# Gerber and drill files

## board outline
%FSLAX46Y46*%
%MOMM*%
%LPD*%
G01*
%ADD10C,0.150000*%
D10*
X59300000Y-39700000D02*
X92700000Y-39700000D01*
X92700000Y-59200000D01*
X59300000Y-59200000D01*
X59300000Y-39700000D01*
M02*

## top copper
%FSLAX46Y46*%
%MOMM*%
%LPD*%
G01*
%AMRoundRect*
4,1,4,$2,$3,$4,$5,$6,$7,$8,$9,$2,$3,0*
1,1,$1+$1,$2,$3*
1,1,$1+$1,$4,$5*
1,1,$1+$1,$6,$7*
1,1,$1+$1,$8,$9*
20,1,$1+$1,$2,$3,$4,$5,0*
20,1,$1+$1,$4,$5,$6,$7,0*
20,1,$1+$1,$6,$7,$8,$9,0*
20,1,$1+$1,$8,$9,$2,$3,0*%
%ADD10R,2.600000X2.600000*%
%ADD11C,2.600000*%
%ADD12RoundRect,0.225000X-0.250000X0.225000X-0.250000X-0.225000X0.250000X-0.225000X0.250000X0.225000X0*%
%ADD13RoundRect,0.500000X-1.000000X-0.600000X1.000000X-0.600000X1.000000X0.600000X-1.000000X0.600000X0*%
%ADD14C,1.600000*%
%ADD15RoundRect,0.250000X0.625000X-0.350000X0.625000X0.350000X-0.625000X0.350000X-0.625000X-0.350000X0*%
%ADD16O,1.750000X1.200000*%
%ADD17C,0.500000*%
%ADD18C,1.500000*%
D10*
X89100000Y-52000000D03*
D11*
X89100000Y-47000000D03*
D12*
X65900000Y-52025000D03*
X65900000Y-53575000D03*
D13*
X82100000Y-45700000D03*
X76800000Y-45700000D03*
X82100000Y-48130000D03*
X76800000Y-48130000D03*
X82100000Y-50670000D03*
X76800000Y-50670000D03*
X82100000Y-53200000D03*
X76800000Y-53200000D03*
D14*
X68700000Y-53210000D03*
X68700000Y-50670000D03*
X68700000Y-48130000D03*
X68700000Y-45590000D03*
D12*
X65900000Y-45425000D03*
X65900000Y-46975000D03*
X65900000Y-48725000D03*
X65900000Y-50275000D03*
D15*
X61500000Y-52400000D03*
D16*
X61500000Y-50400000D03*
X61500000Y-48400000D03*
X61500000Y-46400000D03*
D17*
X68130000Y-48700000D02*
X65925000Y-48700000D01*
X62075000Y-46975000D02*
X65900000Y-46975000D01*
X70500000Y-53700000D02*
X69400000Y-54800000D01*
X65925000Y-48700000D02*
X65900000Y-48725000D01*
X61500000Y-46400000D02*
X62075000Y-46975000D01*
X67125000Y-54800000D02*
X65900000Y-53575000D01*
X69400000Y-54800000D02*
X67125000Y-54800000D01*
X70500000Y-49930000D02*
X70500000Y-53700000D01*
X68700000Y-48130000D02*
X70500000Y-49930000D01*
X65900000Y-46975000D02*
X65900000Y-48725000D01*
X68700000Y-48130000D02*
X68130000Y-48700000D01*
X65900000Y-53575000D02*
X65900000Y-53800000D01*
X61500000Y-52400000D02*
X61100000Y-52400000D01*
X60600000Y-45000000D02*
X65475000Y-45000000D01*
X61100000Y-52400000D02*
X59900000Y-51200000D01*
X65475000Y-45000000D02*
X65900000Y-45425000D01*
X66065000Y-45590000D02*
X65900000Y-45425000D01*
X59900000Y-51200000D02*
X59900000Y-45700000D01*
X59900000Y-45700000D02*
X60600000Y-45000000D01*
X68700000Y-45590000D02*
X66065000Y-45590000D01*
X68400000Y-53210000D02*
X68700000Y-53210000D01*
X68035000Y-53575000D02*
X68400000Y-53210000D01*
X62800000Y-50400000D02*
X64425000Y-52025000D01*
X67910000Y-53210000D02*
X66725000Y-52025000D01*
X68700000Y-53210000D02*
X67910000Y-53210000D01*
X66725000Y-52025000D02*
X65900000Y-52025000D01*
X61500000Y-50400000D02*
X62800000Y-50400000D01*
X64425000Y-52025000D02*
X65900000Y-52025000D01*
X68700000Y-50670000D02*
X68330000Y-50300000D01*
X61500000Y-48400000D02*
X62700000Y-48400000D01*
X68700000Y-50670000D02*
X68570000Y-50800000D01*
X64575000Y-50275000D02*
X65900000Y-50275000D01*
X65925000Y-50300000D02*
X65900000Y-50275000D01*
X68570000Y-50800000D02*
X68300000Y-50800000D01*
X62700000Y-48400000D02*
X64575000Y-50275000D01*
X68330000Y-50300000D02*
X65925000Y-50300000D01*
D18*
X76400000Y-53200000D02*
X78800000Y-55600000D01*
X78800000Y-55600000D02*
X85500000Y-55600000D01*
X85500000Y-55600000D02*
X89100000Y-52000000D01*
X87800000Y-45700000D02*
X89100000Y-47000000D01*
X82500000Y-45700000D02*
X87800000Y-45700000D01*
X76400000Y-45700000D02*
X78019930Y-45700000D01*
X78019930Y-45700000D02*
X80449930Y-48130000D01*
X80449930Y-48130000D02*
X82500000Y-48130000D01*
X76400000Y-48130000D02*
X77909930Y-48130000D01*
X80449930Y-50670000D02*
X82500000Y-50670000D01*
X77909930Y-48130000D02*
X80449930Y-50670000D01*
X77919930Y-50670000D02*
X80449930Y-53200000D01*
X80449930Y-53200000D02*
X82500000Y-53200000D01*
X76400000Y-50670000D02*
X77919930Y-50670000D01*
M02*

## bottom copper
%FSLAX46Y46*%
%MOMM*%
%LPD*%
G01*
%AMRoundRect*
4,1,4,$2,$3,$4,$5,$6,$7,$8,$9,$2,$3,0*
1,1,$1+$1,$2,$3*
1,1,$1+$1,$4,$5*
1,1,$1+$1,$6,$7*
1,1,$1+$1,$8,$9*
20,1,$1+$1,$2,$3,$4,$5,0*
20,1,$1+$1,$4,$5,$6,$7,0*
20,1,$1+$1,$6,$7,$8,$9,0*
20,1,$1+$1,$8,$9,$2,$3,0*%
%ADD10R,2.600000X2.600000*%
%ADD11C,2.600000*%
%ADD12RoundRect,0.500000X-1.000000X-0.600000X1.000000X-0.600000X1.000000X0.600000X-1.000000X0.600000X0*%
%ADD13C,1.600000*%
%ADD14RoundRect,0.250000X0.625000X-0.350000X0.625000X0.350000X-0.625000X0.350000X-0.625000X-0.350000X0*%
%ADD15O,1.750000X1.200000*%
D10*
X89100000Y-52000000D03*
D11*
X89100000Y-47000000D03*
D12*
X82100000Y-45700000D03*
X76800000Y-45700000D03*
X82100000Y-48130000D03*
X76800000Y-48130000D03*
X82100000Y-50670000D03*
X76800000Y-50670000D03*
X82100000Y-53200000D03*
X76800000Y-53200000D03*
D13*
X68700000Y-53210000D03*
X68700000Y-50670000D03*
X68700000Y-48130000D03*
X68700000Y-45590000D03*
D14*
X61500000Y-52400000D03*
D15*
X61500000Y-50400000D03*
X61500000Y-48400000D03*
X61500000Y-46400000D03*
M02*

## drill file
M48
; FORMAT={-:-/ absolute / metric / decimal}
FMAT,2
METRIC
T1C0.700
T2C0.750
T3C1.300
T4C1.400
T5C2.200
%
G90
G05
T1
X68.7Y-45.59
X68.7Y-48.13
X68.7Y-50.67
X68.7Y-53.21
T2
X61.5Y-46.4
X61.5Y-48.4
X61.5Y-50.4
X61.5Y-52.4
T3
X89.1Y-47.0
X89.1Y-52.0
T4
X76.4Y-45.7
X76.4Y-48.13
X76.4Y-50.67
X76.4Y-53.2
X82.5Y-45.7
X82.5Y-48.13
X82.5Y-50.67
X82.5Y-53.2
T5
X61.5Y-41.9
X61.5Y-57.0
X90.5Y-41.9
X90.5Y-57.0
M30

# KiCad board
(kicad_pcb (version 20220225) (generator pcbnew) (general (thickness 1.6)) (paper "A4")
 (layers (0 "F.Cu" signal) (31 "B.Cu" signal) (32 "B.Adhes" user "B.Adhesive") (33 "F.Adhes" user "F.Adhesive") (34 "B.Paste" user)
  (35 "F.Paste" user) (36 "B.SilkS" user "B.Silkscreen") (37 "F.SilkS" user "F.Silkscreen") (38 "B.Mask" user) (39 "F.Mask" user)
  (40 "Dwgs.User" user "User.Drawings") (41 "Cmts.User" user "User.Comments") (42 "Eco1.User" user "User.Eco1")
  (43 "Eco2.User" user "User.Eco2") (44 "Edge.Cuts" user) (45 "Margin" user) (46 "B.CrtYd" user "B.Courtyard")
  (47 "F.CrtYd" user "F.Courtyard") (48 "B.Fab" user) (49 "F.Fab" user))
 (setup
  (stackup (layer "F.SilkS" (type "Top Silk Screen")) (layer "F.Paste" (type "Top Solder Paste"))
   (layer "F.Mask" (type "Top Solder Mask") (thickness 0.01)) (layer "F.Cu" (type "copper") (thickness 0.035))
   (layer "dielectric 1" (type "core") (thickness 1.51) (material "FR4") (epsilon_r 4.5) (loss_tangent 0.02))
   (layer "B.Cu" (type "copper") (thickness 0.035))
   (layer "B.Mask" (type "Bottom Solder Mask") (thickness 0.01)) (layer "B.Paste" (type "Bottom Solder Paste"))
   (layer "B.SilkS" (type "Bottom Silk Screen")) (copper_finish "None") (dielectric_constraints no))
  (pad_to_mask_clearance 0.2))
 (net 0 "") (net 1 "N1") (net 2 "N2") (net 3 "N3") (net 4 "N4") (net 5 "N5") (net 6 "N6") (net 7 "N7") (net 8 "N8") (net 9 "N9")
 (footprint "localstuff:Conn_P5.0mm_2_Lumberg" (layer "F.Cu") (at 89.1 52 90)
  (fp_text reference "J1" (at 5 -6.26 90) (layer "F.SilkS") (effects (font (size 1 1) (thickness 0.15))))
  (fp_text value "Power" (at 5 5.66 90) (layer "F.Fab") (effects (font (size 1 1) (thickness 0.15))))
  (pad "1" thru_hole rect (at 0 0 90) (size 2.6 2.6) (drill 1.3) (layers *.Cu *.Mask) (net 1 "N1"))
  (pad "2" thru_hole circle (at 5 0 90) (size 2.6 2.6) (drill 1.3) (layers *.Cu *.Mask) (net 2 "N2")))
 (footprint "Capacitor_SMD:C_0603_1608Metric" (layer "F.Cu") (at 65.9 52.8 -90)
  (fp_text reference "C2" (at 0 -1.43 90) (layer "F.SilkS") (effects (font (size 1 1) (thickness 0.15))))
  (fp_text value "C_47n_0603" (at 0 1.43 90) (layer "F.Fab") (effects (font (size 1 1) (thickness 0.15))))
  (pad "1" smd roundrect (at -0.775 0 270) (size 0.9 0.95) (layers "F.Cu" "F.Paste" "F.Mask") (roundrect_rratio 0.25) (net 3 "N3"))
  (pad "2" smd roundrect (at 0.775 0 270) (size 0.9 0.95) (layers "F.Cu" "F.Paste" "F.Mask") (roundrect_rratio 0.25) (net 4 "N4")))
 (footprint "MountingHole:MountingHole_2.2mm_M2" (layer "F.Cu") (at 90.5 41.9)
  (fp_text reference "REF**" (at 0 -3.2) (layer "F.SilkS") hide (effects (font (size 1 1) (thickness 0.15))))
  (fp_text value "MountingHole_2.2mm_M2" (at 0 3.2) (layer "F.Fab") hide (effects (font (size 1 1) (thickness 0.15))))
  (pad "" np_thru_hole circle (at 0 0) (size 2.2 2.2) (drill 2.2) (layers F&B.Cu *.Mask)))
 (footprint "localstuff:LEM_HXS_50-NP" (layer "F.Cu") (at 75.8 49.4)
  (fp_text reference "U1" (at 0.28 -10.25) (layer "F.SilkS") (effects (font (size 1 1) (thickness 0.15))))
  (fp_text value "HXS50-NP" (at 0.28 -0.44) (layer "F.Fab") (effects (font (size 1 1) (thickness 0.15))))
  (pad "1" thru_hole roundrect (at 6.7 -3.7) (size 3 2.2) (drill 1.4 (offset -0.4 0)) (layers *.Cu *.Mask) (roundrect_rratio 0.2272727273)
   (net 2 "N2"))
  (pad "2" thru_hole roundrect (at 0.6 -3.7) (size 3 2.2) (drill 1.4 (offset 0.4 0)) (layers *.Cu *.Mask) (roundrect_rratio 0.2272727273)
   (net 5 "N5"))
  (pad "3" thru_hole roundrect (at 6.7 -1.27) (size 3 2.2) (drill 1.4 (offset -0.4 0)) (layers *.Cu *.Mask) (roundrect_rratio 0.2272727273)
   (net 5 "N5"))
  (pad "4" thru_hole roundrect (at 0.6 -1.27) (size 3 2.2) (drill 1.4 (offset 0.4 0)) (layers *.Cu *.Mask) (roundrect_rratio 0.2272727273)
   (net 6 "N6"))
  (pad "5" thru_hole roundrect (at 6.7 1.27) (size 3 2.2) (drill 1.4 (offset -0.4 0)) (layers *.Cu *.Mask) (roundrect_rratio 0.2272727273)
   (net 6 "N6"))
  (pad "6" thru_hole roundrect (at 0.6 1.27) (size 3 2.2) (drill 1.4 (offset 0.4 0)) (layers *.Cu *.Mask) (roundrect_rratio 0.2272727273)
   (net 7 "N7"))
  (pad "7" thru_hole roundrect (at 6.7 3.8) (size 3 2.2) (drill 1.4 (offset -0.4 0)) (layers *.Cu *.Mask) (roundrect_rratio 0.2272727273)
   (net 7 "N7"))
  (pad "8" thru_hole roundrect (at 0.6 3.8) (size 3 2.2) (drill 1.4 (offset 0.4 0)) (layers *.Cu *.Mask) (roundrect_rratio 0.2272727273)
   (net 1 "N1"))
  (pad "9" thru_hole circle (at -7.1 3.81) (size 1.6 1.6) (drill 0.7) (layers *.Cu *.Mask) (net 3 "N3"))
  (pad "10" thru_hole circle (at -7.1 1.27) (size 1.6 1.6) (drill 0.7) (layers *.Cu *.Mask) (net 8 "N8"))
  (pad "11" thru_hole circle (at -7.1 -1.27 90) (size 1.6 1.6) (drill 0.7) (layers *.Cu *.Mask) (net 4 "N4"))
  (pad "12" thru_hole circle (at -7.1 -3.81) (size 1.6 1.6) (drill 0.7) (layers *.Cu *.Mask) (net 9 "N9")))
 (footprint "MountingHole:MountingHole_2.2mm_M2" (layer "F.Cu") (at 61.5 57)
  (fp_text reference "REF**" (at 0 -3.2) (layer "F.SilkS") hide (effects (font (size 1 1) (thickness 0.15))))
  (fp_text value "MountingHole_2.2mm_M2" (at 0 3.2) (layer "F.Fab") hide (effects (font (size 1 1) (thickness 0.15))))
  (pad "" np_thru_hole circle (at 0 0) (size 2.2 2.2) (drill 2.2) (layers F&B.Cu *.Mask)))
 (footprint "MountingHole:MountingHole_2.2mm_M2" (layer "F.Cu") (at 90.5 57)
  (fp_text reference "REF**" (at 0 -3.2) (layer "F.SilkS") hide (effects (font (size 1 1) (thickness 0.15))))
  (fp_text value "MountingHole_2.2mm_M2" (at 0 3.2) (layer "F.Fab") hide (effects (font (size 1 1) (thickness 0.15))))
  (pad "" np_thru_hole circle (at 0 0) (size 2.2 2.2) (drill 2.2) (layers F&B.Cu *.Mask)))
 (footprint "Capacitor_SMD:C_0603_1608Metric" (layer "F.Cu") (at 65.9 46.2 -90)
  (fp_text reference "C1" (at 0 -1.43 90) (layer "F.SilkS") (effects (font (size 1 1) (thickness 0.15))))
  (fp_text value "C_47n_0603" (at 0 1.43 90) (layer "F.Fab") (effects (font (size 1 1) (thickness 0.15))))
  (pad "1" smd roundrect (at -0.775 0 270) (size 0.9 0.95) (layers "F.Cu" "F.Paste" "F.Mask") (roundrect_rratio 0.25) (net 9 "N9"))
  (pad "2" smd roundrect (at 0.775 0 270) (size 0.9 0.95) (layers "F.Cu" "F.Paste" "F.Mask") (roundrect_rratio 0.25) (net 4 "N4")))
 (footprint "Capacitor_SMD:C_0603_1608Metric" (layer "F.Cu") (at 65.9 49.5 -90)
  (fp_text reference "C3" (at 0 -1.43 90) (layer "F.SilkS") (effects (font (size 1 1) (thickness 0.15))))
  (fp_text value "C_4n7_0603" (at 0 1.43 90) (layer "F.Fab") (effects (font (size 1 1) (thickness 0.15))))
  (pad "1" smd roundrect (at -0.775 0 270) (size 0.9 0.95) (layers "F.Cu" "F.Paste" "F.Mask") (roundrect_rratio 0.25) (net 4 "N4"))
  (pad "2" smd roundrect (at 0.775 0 270) (size 0.9 0.95) (layers "F.Cu" "F.Paste" "F.Mask") (roundrect_rratio 0.25) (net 8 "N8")))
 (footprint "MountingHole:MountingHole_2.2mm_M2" (layer "F.Cu") (at 61.5 41.9)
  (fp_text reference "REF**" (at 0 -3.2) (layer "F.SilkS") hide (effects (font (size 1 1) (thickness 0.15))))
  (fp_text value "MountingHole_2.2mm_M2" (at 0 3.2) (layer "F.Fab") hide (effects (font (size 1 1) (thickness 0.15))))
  (pad "" np_thru_hole circle (at 0 0) (size 2.2 2.2) (drill 2.2) (layers F&B.Cu *.Mask)))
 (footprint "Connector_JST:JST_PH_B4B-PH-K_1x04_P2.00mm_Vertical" (layer "F.Cu") (at 61.5 52.4 90)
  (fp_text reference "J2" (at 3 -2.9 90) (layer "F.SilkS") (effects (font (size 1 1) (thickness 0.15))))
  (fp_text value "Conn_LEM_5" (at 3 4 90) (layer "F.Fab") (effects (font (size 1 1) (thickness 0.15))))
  (pad "1" thru_hole roundrect (at 0 0 90) (size 1.2 1.75) (drill 0.75) (layers *.Cu *.Mask) (roundrect_rratio 0.2083333333) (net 9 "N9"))
  (pad "2" thru_hole oval (at 2 0 90) (size 1.2 1.75) (drill 0.75) (layers *.Cu *.Mask) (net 3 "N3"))
  (pad "3" thru_hole oval (at 4 0 90) (size 1.2 1.75) (drill 0.75) (layers *.Cu *.Mask) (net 8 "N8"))
  (pad "4" thru_hole oval (at 6 0 90) (size 1.2 1.75) (drill 0.75) (layers *.Cu *.Mask) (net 4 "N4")))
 (gr_rect (start 59.3 39.7) (end 92.7 59.2) (stroke (width 0.15) (type default)) (fill none) (layer "Edge.Cuts"))
 (segment (start 68.13 48.7) (end 65.925 48.7) (width 0.5) (layer "F.Cu") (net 4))
 (segment (start 62.075 46.975) (end 65.9 46.975) (width 0.5) (layer "F.Cu") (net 4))
 (segment (start 70.5 53.7) (end 69.4 54.8) (width 0.5) (layer "F.Cu") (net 4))
 (segment (start 65.925 48.7) (end 65.9 48.725) (width 0.5) (layer "F.Cu") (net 4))
 (segment (start 61.5 46.4) (end 62.075 46.975) (width 0.5) (layer "F.Cu") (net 4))
 (segment (start 67.125 54.8) (end 65.9 53.575) (width 0.5) (layer "F.Cu") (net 4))
 (segment (start 69.4 54.8) (end 67.125 54.8) (width 0.5) (layer "F.Cu") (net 4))
 (segment (start 70.5 49.93) (end 70.5 53.7) (width 0.5) (layer "F.Cu") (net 4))
 (segment (start 68.7 48.13) (end 70.5 49.93) (width 0.5) (layer "F.Cu") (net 4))
 (segment (start 65.9 46.975) (end 65.9 48.725) (width 0.5) (layer "F.Cu") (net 4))
 (segment (start 68.7 48.13) (end 68.13 48.7) (width 0.5) (layer "F.Cu") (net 4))
 (segment (start 65.9 53.575) (end 65.9 53.8) (width 0.5) (layer "F.Cu") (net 4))
 (segment (start 61.5 52.4) (end 61.1 52.4) (width 0.5) (layer "F.Cu") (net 9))
 (segment (start 60.6 45) (end 65.475 45) (width 0.5) (layer "F.Cu") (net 9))
 (segment (start 61.1 52.4) (end 59.9 51.2) (width 0.5) (layer "F.Cu") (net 9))
 (segment (start 65.475 45) (end 65.9 45.425) (width 0.5) (layer "F.Cu") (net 9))
 (segment (start 66.065 45.59) (end 65.9 45.425) (width 0.5) (layer "F.Cu") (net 9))
 (segment (start 59.9 51.2) (end 59.9 45.7) (width 0.5) (layer "F.Cu") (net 9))
 (segment (start 59.9 45.7) (end 60.6 45) (width 0.5) (layer "F.Cu") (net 9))
 (segment (start 68.7 45.59) (end 66.065 45.59) (width 0.5) (layer "F.Cu") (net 9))
 (segment (start 68.4 53.21) (end 68.7 53.21) (width 0.5) (layer "F.Cu") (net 3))
 (segment (start 68.035 53.575) (end 68.4 53.21) (width 0.5) (layer "F.Cu") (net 3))
 (segment (start 62.8 50.4) (end 64.425 52.025) (width 0.5) (layer "F.Cu") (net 3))
 (segment (start 67.91 53.21) (end 66.725 52.025) (width 0.5) (layer "F.Cu") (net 3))
 (segment (start 68.7 53.21) (end 67.91 53.21) (width 0.5) (layer "F.Cu") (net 3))
 (segment (start 66.725 52.025) (end 65.9 52.025) (width 0.5) (layer "F.Cu") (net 3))
 (segment (start 61.5 50.4) (end 62.8 50.4) (width 0.5) (layer "F.Cu") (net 3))
 (segment (start 64.425 52.025) (end 65.9 52.025) (width 0.5) (layer "F.Cu") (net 3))
 (segment (start 68.7 50.67) (end 68.33 50.3) (width 0.5) (layer "F.Cu") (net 8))
 (segment (start 61.5 48.4) (end 62.7 48.4) (width 0.5) (layer "F.Cu") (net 8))
 (segment (start 68.7 50.67) (end 68.57 50.8) (width 0.5) (layer "F.Cu") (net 8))
 (segment (start 64.575 50.275) (end 65.9 50.275) (width 0.5) (layer "F.Cu") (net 8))
 (segment (start 65.925 50.3) (end 65.9 50.275) (width 0.5) (layer "F.Cu") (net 8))
 (segment (start 68.57 50.8) (end 68.3 50.8) (width 0.5) (layer "F.Cu") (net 8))
 (segment (start 62.7 48.4) (end 64.575 50.275) (width 0.5) (layer "F.Cu") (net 8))
 (segment (start 68.33 50.3) (end 65.925 50.3) (width 0.5) (layer "F.Cu") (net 8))
 (segment (start 76.4 53.2) (end 78.8 55.6) (width 1.5) (layer "F.Cu") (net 1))
 (segment (start 78.8 55.6) (end 85.5 55.6) (width 1.5) (layer "F.Cu") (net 1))
 (segment (start 85.5 55.6) (end 89.1 52) (width 1.5) (layer "F.Cu") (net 1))
 (segment (start 87.8 45.7) (end 89.1 47) (width 1.5) (layer "F.Cu") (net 2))
 (segment (start 82.5 45.7) (end 87.8 45.7) (width 1.5) (layer "F.Cu") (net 2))
 (segment (start 76.4 45.7) (end 78.01993 45.7) (width 1.5) (layer "F.Cu") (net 5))
 (segment (start 78.01993 45.7) (end 80.44993 48.13) (width 1.5) (layer "F.Cu") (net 5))
 (segment (start 80.44993 48.13) (end 82.5 48.13) (width 1.5) (layer "F.Cu") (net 5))
 (segment (start 76.4 48.13) (end 77.90993 48.13) (width 1.5) (layer "F.Cu") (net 6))
 (segment (start 80.44993 50.67) (end 82.5 50.67) (width 1.5) (layer "F.Cu") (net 6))
 (segment (start 77.90993 48.13) (end 80.44993 50.67) (width 1.5) (layer "F.Cu") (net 6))
 (segment (start 77.91993 50.67) (end 80.44993 53.2) (width 1.5) (layer "F.Cu") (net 7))
 (segment (start 80.44993 53.2) (end 82.5 53.2) (width 1.5) (layer "F.Cu") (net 7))
 (segment (start 76.4 50.67) (end 77.91993 50.67) (width 1.5) (layer "F.Cu") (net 7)))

